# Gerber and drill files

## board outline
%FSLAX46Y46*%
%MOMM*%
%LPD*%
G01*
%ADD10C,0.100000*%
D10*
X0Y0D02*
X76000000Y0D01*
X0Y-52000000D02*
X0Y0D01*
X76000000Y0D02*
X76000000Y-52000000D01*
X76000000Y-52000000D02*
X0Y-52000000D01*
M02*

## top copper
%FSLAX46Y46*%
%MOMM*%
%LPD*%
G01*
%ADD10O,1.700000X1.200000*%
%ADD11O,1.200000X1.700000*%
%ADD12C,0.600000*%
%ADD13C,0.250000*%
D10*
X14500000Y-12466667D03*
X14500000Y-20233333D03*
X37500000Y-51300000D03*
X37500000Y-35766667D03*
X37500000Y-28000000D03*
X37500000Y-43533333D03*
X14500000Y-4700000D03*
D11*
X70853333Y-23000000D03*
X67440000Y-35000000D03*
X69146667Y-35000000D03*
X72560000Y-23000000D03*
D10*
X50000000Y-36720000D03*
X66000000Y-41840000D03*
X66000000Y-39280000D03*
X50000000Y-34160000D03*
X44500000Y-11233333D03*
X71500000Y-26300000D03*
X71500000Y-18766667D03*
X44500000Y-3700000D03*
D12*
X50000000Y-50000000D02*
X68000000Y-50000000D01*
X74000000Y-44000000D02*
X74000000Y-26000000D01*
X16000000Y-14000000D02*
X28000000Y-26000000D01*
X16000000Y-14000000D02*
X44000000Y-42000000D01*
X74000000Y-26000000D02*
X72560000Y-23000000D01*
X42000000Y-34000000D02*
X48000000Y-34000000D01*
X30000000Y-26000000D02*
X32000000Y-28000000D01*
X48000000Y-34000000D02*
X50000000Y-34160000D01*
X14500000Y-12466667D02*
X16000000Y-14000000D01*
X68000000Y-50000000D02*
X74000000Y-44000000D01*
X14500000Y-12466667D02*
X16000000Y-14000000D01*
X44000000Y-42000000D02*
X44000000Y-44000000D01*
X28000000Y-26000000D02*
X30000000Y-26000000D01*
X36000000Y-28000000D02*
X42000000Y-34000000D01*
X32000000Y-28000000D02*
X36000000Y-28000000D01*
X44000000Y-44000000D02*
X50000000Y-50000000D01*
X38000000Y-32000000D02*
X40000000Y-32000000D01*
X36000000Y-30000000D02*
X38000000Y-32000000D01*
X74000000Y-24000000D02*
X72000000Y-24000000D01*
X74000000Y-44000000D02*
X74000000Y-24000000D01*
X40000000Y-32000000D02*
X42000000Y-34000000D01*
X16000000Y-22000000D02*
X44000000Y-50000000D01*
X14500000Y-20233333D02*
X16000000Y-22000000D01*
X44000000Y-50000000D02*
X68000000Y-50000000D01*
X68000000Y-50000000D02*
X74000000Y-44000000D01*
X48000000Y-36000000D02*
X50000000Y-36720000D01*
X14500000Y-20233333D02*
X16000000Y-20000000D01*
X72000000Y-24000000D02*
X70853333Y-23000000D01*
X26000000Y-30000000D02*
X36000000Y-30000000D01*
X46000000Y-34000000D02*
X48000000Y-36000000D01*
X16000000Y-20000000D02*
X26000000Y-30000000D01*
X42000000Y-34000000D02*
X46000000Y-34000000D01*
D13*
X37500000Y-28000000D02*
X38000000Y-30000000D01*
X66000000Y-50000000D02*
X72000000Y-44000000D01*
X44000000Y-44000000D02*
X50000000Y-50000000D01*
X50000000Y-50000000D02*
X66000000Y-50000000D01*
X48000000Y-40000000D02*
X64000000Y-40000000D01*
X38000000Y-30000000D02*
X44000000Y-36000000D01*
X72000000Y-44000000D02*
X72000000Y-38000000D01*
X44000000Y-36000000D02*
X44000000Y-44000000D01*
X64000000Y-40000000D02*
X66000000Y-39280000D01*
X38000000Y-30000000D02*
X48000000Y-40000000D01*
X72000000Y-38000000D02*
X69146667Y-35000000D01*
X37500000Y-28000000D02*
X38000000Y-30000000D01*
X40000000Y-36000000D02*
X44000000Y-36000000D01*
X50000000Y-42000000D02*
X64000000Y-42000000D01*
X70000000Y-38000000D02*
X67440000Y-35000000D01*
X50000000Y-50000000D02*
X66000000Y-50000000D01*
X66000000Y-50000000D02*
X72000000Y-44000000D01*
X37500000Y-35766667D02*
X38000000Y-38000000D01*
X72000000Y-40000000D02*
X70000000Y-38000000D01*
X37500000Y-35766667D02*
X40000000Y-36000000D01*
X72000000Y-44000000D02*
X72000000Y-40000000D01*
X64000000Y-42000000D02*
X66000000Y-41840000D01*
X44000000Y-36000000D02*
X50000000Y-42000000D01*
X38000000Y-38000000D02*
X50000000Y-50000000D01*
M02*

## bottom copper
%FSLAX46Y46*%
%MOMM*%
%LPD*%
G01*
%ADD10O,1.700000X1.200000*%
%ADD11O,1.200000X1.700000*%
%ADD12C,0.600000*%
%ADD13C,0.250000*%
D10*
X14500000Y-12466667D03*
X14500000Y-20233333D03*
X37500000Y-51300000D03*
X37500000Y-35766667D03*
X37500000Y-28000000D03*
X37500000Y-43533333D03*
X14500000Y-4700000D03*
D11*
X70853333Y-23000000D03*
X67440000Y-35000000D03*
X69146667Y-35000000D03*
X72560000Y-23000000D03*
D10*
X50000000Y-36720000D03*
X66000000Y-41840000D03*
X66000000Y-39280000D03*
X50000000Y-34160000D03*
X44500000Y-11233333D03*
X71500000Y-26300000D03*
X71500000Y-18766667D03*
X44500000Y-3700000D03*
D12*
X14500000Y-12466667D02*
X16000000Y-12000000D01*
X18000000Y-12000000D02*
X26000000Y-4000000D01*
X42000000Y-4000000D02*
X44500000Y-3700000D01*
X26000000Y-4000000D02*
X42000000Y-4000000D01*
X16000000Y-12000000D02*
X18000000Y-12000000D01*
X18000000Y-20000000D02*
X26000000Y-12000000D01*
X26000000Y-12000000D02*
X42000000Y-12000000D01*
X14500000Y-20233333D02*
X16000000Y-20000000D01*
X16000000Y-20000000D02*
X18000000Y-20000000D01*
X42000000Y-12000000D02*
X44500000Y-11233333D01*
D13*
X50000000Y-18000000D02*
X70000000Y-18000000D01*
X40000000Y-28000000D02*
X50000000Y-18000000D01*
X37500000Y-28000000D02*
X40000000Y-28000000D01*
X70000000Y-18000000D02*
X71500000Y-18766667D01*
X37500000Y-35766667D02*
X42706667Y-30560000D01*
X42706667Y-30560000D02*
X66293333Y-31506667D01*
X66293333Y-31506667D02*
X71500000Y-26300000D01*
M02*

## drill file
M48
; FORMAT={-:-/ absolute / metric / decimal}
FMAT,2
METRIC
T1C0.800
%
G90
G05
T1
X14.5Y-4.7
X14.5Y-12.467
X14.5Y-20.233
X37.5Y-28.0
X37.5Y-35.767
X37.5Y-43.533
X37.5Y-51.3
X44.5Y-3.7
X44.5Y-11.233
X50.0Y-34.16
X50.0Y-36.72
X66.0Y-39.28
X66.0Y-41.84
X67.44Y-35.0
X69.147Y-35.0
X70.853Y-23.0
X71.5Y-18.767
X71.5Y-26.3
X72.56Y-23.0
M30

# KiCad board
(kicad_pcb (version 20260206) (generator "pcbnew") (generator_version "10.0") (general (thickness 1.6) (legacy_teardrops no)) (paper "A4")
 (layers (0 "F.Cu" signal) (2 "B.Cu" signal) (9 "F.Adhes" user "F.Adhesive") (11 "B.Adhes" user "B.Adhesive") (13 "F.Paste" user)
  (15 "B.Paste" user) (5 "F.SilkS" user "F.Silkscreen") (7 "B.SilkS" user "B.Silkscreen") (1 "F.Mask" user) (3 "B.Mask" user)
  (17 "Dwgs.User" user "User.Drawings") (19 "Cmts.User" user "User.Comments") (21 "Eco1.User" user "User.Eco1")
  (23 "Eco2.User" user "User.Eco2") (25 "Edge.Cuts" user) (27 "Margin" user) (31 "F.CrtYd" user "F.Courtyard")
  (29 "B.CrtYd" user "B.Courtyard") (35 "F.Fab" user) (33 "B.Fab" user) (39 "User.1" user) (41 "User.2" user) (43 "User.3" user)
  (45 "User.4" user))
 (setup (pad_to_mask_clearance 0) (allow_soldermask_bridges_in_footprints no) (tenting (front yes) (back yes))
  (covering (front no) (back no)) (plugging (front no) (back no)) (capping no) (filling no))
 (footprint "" (layer "F.Cu") (at 26 28)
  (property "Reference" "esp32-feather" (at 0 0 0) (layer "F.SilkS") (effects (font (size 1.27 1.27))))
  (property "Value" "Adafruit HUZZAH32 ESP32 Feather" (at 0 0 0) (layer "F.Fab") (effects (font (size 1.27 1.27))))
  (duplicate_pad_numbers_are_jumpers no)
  (pad "3V3" thru_hole oval (at -11.5 -15.533333) (size 1.7 1.2) (drill 0.8) (layers "*.Cu") (remove_unused_layers no) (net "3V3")
   (thermal_bridge_angle 45))
  (pad "GND" thru_hole oval (at -11.5 -7.766667) (size 1.7 1.2) (drill 0.8) (layers "*.Cu") (remove_unused_layers no) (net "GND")
   (thermal_bridge_angle 45))
  (pad "RX" thru_hole oval (at 11.5 23.3) (size 1.7 1.2) (drill 0.8) (layers "*.Cu") (remove_unused_layers no) (thermal_bridge_angle 45))
  (pad "SCL" thru_hole oval (at 11.5 7.766667) (size 1.7 1.2) (drill 0.8) (layers "*.Cu") (remove_unused_layers no) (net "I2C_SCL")
   (thermal_bridge_angle 45))
  (pad "SDA" thru_hole oval (at 11.5 0) (size 1.7 1.2) (drill 0.8) (layers "*.Cu") (remove_unused_layers no) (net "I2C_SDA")
   (thermal_bridge_angle 45))
  (pad "TX" thru_hole oval (at 11.5 15.533333) (size 1.7 1.2) (drill 0.8) (layers "*.Cu") (remove_unused_layers no)
   (thermal_bridge_angle 45))
  (pad "VIN" thru_hole oval (at -11.5 -23.3) (size 1.7 1.2) (drill 0.8) (layers "*.Cu") (remove_unused_layers no) (thermal_bridge_angle 45)))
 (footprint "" (layer "F.Cu") (at 70 29 90)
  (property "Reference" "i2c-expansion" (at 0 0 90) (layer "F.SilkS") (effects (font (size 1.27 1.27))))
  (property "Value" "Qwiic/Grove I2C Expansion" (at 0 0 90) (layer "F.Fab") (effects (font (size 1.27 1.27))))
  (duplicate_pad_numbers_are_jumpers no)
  (pad "GND" thru_hole oval (at 6 0.853333 90) (size 1.7 1.2) (drill 0.8) (layers "*.Cu") (remove_unused_layers no) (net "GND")
   (thermal_bridge_angle 45))
  (pad "SCL" thru_hole oval (at -6 -2.56 90) (size 1.7 1.2) (drill 0.8) (layers "*.Cu") (remove_unused_layers no) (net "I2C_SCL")
   (thermal_bridge_angle 45))
  (pad "SDA" thru_hole oval (at -6 -0.853333 90) (size 1.7 1.2) (drill 0.8) (layers "*.Cu") (remove_unused_layers no) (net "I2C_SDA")
   (thermal_bridge_angle 45))
  (pad "VCC" thru_hole oval (at 6 2.56 90) (size 1.7 1.2) (drill 0.8) (layers "*.Cu") (remove_unused_layers no) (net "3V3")
   (thermal_bridge_angle 45)))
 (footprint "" (layer "F.Cu") (at 58 38)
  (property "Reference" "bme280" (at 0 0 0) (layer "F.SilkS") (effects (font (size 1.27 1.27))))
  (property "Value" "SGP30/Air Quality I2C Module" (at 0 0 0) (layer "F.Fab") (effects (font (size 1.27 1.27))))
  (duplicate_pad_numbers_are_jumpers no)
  (pad "GND" thru_hole oval (at -8 -1.28) (size 1.7 1.2) (drill 0.8) (layers "*.Cu") (remove_unused_layers no) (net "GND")
   (thermal_bridge_angle 45))
  (pad "SCL" thru_hole oval (at 8 3.84) (size 1.7 1.2) (drill 0.8) (layers "*.Cu") (remove_unused_layers no) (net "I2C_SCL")
   (thermal_bridge_angle 45))
  (pad "SDA" thru_hole oval (at 8 1.28) (size 1.7 1.2) (drill 0.8) (layers "*.Cu") (remove_unused_layers no) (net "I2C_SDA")
   (thermal_bridge_angle 45))
  (pad "VCC" thru_hole oval (at -8 -3.84) (size 1.7 1.2) (drill 0.8) (layers "*.Cu") (remove_unused_layers no) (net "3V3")
   (thermal_bridge_angle 45)))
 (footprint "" (layer "F.Cu") (at 58 15)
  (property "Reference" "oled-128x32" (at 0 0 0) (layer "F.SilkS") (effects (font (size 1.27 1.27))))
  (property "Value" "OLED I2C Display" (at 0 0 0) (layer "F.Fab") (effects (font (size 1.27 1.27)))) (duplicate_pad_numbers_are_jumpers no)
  (pad "GND" thru_hole oval (at -13.5 -3.766667) (size 1.7 1.2) (drill 0.8) (layers "*.Cu") (remove_unused_layers no) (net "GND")
   (thermal_bridge_angle 45))
  (pad "SCL" thru_hole oval (at 13.5 11.3) (size 1.7 1.2) (drill 0.8) (layers "*.Cu") (remove_unused_layers no) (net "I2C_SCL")
   (thermal_bridge_angle 45))
  (pad "SDA" thru_hole oval (at 13.5 3.766667) (size 1.7 1.2) (drill 0.8) (layers "*.Cu") (remove_unused_layers no) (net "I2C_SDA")
   (thermal_bridge_angle 45))
  (pad "VCC" thru_hole oval (at -13.5 -11.3) (size 1.7 1.2) (drill 0.8) (layers "*.Cu") (remove_unused_layers no) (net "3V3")
   (thermal_bridge_angle 45)))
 (gr_line (start 0 0) (end 76 0) (stroke (width 0.1) (type default)) (layer "Edge.Cuts"))
 (gr_line (start 0 52) (end 0 0) (stroke (width 0.1) (type default)) (layer "Edge.Cuts"))
 (gr_line (start 76 0) (end 76 52) (stroke (width 0.1) (type default)) (layer "Edge.Cuts"))
 (gr_line (start 76 52) (end 0 52) (stroke (width 0.1) (type default)) (layer "Edge.Cuts"))
 (segment (start 50 50) (end 68 50) (width 0.6) (layer "F.Cu") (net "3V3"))
 (segment (start 74 44) (end 74 26) (width 0.6) (layer "F.Cu") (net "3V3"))
 (segment (start 16 14) (end 28 26) (width 0.6) (layer "F.Cu") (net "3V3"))
 (segment (start 16 14) (end 44 42) (width 0.6) (layer "F.Cu") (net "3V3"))
 (segment (start 74 26) (end 72.56 23) (width 0.6) (layer "F.Cu") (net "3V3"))
 (segment (start 42 34) (end 48 34) (width 0.6) (layer "F.Cu") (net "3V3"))
 (segment (start 30 26) (end 32 28) (width 0.6) (layer "F.Cu") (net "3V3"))
 (segment (start 48 34) (end 50 34.16) (width 0.6) (layer "F.Cu") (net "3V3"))
 (segment (start 14.5 12.466667) (end 16 14) (width 0.6) (layer "F.Cu") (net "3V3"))
 (segment (start 68 50) (end 74 44) (width 0.6) (layer "F.Cu") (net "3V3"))
 (segment (start 14.5 12.466667) (end 16 14) (width 0.6) (layer "F.Cu") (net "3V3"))
 (segment (start 44 42) (end 44 44) (width 0.6) (layer "F.Cu") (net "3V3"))
 (segment (start 28 26) (end 30 26) (width 0.6) (layer "F.Cu") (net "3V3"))
 (segment (start 36 28) (end 42 34) (width 0.6) (layer "F.Cu") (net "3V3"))
 (segment (start 32 28) (end 36 28) (width 0.6) (layer "F.Cu") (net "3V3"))
 (segment (start 44 44) (end 50 50) (width 0.6) (layer "F.Cu") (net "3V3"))
 (segment (start 14.5 12.466667) (end 16 12) (width 0.6) (layer "B.Cu") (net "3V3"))
 (segment (start 18 12) (end 26 4) (width 0.6) (layer "B.Cu") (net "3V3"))
 (segment (start 42 4) (end 44.5 3.7) (width 0.6) (layer "B.Cu") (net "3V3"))
 (segment (start 26 4) (end 42 4) (width 0.6) (layer "B.Cu") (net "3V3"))
 (segment (start 16 12) (end 18 12) (width 0.6) (layer "B.Cu") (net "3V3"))
 (segment (start 38 32) (end 40 32) (width 0.6) (layer "F.Cu") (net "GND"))
 (segment (start 36 30) (end 38 32) (width 0.6) (layer "F.Cu") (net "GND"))
 (segment (start 74 24) (end 72 24) (width 0.6) (layer "F.Cu") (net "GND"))
 (segment (start 74 44) (end 74 24) (width 0.6) (layer "F.Cu") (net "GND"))
 (segment (start 40 32) (end 42 34) (width 0.6) (layer "F.Cu") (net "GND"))
 (segment (start 16 22) (end 44 50) (width 0.6) (layer "F.Cu") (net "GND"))
 (segment (start 14.5 20.233333) (end 16 22) (width 0.6) (layer "F.Cu") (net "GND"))
 (segment (start 44 50) (end 68 50) (width 0.6) (layer "F.Cu") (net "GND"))
 (segment (start 68 50) (end 74 44) (width 0.6) (layer "F.Cu") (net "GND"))
 (segment (start 48 36) (end 50 36.72) (width 0.6) (layer "F.Cu") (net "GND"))
 (segment (start 14.5 20.233333) (end 16 20) (width 0.6) (layer "F.Cu") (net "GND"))
 (segment (start 72 24) (end 70.853333 23) (width 0.6) (layer "F.Cu") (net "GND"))
 (segment (start 26 30) (end 36 30) (width 0.6) (layer "F.Cu") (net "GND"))
 (segment (start 46 34) (end 48 36) (width 0.6) (layer "F.Cu") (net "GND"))
 (segment (start 16 20) (end 26 30) (width 0.6) (layer "F.Cu") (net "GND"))
 (segment (start 42 34) (end 46 34) (width 0.6) (layer "F.Cu") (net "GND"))
 (segment (start 18 20) (end 26 12) (width 0.6) (layer "B.Cu") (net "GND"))
 (segment (start 26 12) (end 42 12) (width 0.6) (layer "B.Cu") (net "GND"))
 (segment (start 14.5 20.233333) (end 16 20) (width 0.6) (layer "B.Cu") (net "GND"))
 (segment (start 16 20) (end 18 20) (width 0.6) (layer "B.Cu") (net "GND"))
 (segment (start 42 12) (end 44.5 11.233333) (width 0.6) (layer "B.Cu") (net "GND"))
 (segment (start 37.5 28) (end 38 30) (width 0.25) (layer "F.Cu") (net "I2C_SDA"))
 (segment (start 66 50) (end 72 44) (width 0.25) (layer "F.Cu") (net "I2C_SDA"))
 (segment (start 44 44) (end 50 50) (width 0.25) (layer "F.Cu") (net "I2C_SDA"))
 (segment (start 50 50) (end 66 50) (width 0.25) (layer "F.Cu") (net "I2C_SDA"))
 (segment (start 48 40) (end 64 40) (width 0.25) (layer "F.Cu") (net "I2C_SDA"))
 (segment (start 38 30) (end 44 36) (width 0.25) (layer "F.Cu") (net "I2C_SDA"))
 (segment (start 72 44) (end 72 38) (width 0.25) (layer "F.Cu") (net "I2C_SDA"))
 (segment (start 44 36) (end 44 44) (width 0.25) (layer "F.Cu") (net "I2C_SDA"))
 (segment (start 64 40) (end 66 39.28) (width 0.25) (layer "F.Cu") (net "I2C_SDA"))
 (segment (start 38 30) (end 48 40) (width 0.25) (layer "F.Cu") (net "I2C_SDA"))
 (segment (start 72 38) (end 69.146667 35) (width 0.25) (layer "F.Cu") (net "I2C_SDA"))
 (segment (start 37.5 28) (end 38 30) (width 0.25) (layer "F.Cu") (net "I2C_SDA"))
 (segment (start 50 18) (end 70 18) (width 0.25) (layer "B.Cu") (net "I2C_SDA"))
 (segment (start 40 28) (end 50 18) (width 0.25) (layer "B.Cu") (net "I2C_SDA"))
 (segment (start 37.5 28) (end 40 28) (width 0.25) (layer "B.Cu") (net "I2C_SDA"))
 (segment (start 70 18) (end 71.5 18.766667) (width 0.25) (layer "B.Cu") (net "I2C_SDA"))
 (segment (start 40 36) (end 44 36) (width 0.25) (layer "F.Cu") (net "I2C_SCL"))
 (segment (start 50 42) (end 64 42) (width 0.25) (layer "F.Cu") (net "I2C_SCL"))
 (segment (start 70 38) (end 67.44 35) (width 0.25) (layer "F.Cu") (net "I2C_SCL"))
 (segment (start 50 50) (end 66 50) (width 0.25) (layer "F.Cu") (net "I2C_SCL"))
 (segment (start 66 50) (end 72 44) (width 0.25) (layer "F.Cu") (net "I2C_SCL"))
 (segment (start 37.5 35.766667) (end 38 38) (width 0.25) (layer "F.Cu") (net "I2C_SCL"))
 (segment (start 72 40) (end 70 38) (width 0.25) (layer "F.Cu") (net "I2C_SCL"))
 (segment (start 37.5 35.766667) (end 40 36) (width 0.25) (layer "F.Cu") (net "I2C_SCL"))
 (segment (start 72 44) (end 72 40) (width 0.25) (layer "F.Cu") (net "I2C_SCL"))
 (segment (start 64 42) (end 66 41.84) (width 0.25) (layer "F.Cu") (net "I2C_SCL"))
 (segment (start 44 36) (end 50 42) (width 0.25) (layer "F.Cu") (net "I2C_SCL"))
 (segment (start 38 38) (end 50 50) (width 0.25) (layer "F.Cu") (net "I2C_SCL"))
 (segment (start 37.5 35.766667) (end 42.706667 30.56) (width 0.25) (layer "B.Cu") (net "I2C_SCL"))
 (segment (start 42.706667 30.56) (end 66.293333 31.506667) (width 0.25) (layer "B.Cu") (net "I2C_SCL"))
 (segment (start 66.293333 31.506667) (end 71.5 26.3) (width 0.25) (layer "B.Cu") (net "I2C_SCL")))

